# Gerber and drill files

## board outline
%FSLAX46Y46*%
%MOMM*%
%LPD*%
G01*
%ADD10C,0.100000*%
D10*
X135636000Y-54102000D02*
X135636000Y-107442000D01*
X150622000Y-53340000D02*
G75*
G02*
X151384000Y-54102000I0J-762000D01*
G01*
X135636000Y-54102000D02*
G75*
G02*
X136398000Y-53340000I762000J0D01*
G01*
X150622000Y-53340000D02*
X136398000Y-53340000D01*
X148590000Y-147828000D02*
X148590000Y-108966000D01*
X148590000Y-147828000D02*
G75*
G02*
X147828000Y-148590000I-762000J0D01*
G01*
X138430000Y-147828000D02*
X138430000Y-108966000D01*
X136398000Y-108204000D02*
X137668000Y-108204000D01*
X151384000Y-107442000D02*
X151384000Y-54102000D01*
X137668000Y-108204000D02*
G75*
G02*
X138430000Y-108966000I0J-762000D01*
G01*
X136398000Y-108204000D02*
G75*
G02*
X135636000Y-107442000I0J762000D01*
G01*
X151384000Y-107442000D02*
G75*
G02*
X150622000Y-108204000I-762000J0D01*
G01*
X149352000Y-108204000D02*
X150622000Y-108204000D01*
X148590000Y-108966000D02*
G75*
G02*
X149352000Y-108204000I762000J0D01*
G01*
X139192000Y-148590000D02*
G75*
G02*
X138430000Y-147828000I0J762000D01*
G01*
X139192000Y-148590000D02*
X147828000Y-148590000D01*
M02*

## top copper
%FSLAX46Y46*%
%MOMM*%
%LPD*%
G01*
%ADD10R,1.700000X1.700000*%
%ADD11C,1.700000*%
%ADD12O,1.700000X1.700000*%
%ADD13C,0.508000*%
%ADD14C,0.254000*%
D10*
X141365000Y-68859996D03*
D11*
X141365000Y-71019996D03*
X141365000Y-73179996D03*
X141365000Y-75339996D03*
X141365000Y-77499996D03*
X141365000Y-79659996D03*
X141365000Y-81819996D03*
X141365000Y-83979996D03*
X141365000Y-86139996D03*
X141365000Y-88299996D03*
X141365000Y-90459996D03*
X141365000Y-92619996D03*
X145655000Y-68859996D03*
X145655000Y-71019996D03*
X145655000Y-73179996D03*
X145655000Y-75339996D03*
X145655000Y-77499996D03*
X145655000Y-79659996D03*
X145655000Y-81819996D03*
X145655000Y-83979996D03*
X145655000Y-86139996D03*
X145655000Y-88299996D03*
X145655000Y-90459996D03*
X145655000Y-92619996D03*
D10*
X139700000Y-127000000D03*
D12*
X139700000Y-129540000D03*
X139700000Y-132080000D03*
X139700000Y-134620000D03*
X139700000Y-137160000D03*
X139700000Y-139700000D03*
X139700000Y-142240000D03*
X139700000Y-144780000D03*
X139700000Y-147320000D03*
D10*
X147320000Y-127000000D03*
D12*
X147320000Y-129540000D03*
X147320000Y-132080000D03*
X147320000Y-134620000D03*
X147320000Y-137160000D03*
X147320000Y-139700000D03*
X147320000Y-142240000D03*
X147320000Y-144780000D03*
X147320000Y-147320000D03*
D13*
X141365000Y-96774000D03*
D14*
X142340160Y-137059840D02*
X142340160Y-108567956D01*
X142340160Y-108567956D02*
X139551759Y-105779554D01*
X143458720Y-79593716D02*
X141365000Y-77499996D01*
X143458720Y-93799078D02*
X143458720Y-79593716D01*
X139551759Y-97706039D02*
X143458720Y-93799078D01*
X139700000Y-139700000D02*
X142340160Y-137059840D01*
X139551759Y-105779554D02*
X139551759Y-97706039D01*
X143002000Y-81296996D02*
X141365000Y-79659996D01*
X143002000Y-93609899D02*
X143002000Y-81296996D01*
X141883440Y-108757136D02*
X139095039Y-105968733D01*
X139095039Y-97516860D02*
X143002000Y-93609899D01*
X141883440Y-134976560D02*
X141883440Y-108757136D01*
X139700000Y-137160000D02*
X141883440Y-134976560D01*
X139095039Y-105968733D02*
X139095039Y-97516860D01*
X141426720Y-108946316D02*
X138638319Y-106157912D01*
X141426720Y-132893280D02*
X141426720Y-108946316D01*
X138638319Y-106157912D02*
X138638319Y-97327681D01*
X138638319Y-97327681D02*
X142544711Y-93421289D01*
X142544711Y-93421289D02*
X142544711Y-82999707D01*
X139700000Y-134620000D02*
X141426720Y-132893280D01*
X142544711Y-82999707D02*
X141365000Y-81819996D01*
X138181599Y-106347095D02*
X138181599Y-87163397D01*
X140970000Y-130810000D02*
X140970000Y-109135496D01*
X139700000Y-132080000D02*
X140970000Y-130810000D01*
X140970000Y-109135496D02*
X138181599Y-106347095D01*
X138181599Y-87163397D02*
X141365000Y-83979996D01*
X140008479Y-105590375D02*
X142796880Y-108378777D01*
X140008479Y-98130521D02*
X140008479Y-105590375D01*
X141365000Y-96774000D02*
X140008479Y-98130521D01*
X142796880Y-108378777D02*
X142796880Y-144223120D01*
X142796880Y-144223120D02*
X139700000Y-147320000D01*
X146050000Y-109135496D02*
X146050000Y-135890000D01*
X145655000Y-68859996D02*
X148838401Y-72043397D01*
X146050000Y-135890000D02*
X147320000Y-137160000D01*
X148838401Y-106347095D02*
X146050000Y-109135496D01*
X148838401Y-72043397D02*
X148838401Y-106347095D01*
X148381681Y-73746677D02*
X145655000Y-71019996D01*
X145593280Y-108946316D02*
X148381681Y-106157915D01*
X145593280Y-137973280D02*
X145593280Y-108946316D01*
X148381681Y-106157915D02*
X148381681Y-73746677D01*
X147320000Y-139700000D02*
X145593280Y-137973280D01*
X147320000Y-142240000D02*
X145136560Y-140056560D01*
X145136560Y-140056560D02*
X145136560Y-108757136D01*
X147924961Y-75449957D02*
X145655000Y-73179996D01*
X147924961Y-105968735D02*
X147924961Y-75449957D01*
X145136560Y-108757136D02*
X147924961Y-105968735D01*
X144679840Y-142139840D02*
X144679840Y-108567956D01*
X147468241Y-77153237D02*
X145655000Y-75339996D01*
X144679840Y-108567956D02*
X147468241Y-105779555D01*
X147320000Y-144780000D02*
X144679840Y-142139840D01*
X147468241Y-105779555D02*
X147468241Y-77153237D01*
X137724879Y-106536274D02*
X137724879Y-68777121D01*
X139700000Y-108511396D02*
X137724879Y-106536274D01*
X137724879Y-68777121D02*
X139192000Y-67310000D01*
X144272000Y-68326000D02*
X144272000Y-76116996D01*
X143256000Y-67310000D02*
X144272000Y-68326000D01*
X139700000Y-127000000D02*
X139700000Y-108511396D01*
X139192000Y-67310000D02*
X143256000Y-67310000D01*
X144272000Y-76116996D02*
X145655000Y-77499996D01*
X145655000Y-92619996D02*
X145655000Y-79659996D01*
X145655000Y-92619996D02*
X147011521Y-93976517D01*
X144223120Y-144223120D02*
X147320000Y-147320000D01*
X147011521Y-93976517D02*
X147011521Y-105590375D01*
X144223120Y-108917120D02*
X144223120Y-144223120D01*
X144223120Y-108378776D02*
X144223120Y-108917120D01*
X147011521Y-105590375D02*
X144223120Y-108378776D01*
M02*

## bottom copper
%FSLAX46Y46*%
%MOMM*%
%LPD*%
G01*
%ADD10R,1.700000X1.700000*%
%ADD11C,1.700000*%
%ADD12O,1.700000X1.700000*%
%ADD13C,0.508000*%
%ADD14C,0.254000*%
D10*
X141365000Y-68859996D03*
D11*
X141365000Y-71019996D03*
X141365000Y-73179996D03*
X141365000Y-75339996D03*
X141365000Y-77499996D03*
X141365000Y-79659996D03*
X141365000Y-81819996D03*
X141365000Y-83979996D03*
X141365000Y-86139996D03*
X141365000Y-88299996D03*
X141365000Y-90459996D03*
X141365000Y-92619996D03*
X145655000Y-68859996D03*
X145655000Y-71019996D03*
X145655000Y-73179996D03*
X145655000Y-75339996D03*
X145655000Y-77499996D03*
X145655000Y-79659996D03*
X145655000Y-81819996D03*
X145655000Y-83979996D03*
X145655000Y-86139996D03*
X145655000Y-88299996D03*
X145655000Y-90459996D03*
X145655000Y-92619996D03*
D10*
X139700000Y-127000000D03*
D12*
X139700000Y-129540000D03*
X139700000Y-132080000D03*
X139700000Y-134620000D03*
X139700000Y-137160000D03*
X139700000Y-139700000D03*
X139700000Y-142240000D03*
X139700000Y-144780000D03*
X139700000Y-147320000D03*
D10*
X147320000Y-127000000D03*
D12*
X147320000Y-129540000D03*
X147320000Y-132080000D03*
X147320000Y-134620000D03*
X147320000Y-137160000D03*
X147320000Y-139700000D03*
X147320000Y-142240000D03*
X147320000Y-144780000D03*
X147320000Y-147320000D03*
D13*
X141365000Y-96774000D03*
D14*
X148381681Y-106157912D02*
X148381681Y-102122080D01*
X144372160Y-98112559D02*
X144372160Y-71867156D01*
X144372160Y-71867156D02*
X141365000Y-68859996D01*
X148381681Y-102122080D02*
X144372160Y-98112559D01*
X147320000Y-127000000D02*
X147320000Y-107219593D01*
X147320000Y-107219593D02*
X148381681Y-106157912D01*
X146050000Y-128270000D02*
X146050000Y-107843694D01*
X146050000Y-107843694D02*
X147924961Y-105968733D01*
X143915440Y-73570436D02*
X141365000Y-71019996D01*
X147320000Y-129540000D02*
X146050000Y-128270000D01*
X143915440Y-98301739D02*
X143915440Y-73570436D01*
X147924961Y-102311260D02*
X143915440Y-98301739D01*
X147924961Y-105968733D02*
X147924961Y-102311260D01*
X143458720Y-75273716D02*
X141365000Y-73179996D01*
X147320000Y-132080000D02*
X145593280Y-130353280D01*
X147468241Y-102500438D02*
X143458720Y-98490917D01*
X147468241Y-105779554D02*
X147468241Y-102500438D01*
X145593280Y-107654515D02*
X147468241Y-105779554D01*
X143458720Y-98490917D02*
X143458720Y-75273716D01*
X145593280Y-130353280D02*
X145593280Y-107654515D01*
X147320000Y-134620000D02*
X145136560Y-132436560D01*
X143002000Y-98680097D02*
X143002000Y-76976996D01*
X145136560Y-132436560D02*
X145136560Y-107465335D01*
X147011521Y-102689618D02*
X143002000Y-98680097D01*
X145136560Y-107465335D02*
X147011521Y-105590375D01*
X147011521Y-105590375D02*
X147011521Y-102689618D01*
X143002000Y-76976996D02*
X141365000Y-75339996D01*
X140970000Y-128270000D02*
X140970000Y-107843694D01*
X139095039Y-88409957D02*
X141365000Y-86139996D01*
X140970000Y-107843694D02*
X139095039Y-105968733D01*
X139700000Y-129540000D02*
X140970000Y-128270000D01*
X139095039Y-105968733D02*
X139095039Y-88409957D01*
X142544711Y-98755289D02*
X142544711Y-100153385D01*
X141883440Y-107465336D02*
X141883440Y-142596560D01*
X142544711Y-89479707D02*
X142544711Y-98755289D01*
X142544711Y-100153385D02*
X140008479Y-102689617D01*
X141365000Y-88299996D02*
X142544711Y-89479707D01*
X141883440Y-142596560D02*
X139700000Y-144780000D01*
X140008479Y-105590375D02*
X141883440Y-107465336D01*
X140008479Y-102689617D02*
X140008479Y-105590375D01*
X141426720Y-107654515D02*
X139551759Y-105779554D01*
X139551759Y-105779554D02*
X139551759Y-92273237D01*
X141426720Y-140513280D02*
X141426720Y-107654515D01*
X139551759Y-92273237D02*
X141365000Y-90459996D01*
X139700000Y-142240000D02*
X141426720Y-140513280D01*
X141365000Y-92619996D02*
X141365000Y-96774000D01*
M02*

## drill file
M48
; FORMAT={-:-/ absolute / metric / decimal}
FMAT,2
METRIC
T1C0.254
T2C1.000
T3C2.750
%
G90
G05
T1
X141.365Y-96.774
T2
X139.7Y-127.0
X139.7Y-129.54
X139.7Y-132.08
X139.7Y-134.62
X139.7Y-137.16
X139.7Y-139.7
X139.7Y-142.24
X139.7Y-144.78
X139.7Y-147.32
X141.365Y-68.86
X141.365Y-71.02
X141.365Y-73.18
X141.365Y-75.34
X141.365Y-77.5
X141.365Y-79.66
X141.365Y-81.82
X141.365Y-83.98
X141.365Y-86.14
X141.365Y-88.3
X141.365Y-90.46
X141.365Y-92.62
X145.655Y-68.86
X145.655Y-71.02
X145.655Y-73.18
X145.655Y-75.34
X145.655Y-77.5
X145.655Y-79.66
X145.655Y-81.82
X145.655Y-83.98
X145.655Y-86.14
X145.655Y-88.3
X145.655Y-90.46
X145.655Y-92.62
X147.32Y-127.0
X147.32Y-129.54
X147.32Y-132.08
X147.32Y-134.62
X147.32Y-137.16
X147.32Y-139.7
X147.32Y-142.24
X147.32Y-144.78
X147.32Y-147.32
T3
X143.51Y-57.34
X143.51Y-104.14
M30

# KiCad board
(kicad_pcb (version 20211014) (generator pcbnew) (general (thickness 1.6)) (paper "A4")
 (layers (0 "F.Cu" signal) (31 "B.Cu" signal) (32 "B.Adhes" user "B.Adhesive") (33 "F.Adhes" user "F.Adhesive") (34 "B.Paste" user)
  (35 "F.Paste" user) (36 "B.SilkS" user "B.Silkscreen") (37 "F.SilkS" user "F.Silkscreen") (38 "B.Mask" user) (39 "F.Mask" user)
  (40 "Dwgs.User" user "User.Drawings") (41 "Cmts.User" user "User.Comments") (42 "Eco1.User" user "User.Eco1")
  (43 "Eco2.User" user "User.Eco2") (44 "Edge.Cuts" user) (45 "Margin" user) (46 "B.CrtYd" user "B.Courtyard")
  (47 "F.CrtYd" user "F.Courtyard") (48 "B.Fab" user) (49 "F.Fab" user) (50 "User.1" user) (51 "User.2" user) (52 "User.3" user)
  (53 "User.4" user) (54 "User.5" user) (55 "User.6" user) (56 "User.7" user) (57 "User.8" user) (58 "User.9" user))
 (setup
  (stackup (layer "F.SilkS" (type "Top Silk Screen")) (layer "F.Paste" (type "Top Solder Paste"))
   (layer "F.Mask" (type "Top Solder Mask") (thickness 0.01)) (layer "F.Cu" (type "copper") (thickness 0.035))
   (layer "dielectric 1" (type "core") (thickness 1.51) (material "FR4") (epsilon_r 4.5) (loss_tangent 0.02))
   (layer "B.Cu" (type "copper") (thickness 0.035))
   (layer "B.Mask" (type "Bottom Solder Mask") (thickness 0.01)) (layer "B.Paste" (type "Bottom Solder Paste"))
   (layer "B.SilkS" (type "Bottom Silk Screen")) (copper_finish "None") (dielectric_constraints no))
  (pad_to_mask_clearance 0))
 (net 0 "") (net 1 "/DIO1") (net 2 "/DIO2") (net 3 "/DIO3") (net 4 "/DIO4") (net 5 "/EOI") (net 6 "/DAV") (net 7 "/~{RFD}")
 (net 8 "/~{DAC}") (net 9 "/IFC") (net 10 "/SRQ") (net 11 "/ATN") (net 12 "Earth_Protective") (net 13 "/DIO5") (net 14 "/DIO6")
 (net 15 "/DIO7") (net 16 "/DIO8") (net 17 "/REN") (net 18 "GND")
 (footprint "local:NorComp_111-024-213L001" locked (layer "F.Cu") (at 143.51 80.739996 90)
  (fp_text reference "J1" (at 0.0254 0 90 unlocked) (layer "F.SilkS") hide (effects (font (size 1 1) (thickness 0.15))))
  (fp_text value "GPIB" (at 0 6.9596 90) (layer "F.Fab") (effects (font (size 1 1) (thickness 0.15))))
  (pad "" np_thru_hole circle locked (at -23.4 0 90) (size 2.75 2.75) (drill 2.75) (layers *.Cu *.Mask) (solder_mask_margin 1.75)
   (clearance 2))
  (pad "" np_thru_hole circle locked (at 23.4 0 90) (size 2.75 2.75) (drill 2.75) (layers *.Cu *.Mask) (solder_mask_margin 1.75)
   (clearance 2))
  (pad "1" thru_hole rect locked (at 11.88 -2.145 90) (size 1.7 1.7) (drill 1) (layers *.Cu *.Mask) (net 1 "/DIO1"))
  (pad "2" thru_hole circle locked (at 9.72 -2.145 90) (size 1.7 1.7) (drill 1) (layers *.Cu *.Mask) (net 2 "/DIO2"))
  (pad "3" thru_hole circle locked (at 7.56 -2.145 90) (size 1.7 1.7) (drill 1) (layers *.Cu *.Mask) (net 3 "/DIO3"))
  (pad "4" thru_hole circle locked (at 5.4 -2.145 90) (size 1.7 1.7) (drill 1) (layers *.Cu *.Mask) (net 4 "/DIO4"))
  (pad "5" thru_hole circle locked (at 3.24 -2.145 90) (size 1.7 1.7) (drill 1) (layers *.Cu *.Mask) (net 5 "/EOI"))
  (pad "6" thru_hole circle locked (at 1.08 -2.145 90) (size 1.7 1.7) (drill 1) (layers *.Cu *.Mask) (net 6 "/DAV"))
  (pad "7" thru_hole circle locked (at -1.08 -2.145 90) (size 1.7 1.7) (drill 1) (layers *.Cu *.Mask) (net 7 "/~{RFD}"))
  (pad "8" thru_hole circle locked (at -3.24 -2.145 90) (size 1.7 1.7) (drill 1) (layers *.Cu *.Mask) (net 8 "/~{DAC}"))
  (pad "9" thru_hole circle locked (at -5.4 -2.145 90) (size 1.7 1.7) (drill 1) (layers *.Cu *.Mask) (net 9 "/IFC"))
  (pad "10" thru_hole circle locked (at -7.56 -2.145 90) (size 1.7 1.7) (drill 1) (layers *.Cu *.Mask) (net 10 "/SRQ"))
  (pad "11" thru_hole circle locked (at -9.72 -2.145 90) (size 1.7 1.7) (drill 1) (layers *.Cu *.Mask) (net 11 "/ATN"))
  (pad "12" thru_hole circle locked (at -11.88 -2.145 90) (size 1.7 1.7) (drill 1) (layers *.Cu *.Mask) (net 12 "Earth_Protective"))
  (pad "13" thru_hole circle locked (at 11.88 2.145 90) (size 1.7 1.7) (drill 1) (layers *.Cu *.Mask) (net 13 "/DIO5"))
  (pad "14" thru_hole circle locked (at 9.72 2.145 90) (size 1.7 1.7) (drill 1) (layers *.Cu *.Mask) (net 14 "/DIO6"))
  (pad "15" thru_hole circle locked (at 7.56 2.145 90) (size 1.7 1.7) (drill 1) (layers *.Cu *.Mask) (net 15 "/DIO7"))
  (pad "16" thru_hole circle locked (at 5.4 2.145 90) (size 1.7 1.7) (drill 1) (layers *.Cu *.Mask) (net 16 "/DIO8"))
  (pad "17" thru_hole circle locked (at 3.24 2.145 90) (size 1.7 1.7) (drill 1) (layers *.Cu *.Mask) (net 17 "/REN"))
  (pad "18" thru_hole circle locked (at 1.08 2.145 90) (size 1.7 1.7) (drill 1) (layers *.Cu *.Mask) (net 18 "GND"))
  (pad "19" thru_hole circle locked (at -1.08 2.145 90) (size 1.7 1.7) (drill 1) (layers *.Cu *.Mask) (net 18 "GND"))
  (pad "20" thru_hole circle locked (at -3.24 2.145 90) (size 1.7 1.7) (drill 1) (layers *.Cu *.Mask) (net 18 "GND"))
  (pad "21" thru_hole circle locked (at -5.4 2.145 90) (size 1.7 1.7) (drill 1) (layers *.Cu *.Mask) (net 18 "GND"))
  (pad "22" thru_hole circle locked (at -7.56 2.145 90) (size 1.7 1.7) (drill 1) (layers *.Cu *.Mask) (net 18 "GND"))
  (pad "23" thru_hole circle locked (at -9.72 2.145 90) (size 1.7 1.7) (drill 1) (layers *.Cu *.Mask) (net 18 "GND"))
  (pad "24" thru_hole circle locked (at -11.88 2.145 90) (size 1.7 1.7) (drill 1) (layers *.Cu *.Mask) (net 18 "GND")))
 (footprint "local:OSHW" (layer "F.Cu") (at 142.24 122.936 90)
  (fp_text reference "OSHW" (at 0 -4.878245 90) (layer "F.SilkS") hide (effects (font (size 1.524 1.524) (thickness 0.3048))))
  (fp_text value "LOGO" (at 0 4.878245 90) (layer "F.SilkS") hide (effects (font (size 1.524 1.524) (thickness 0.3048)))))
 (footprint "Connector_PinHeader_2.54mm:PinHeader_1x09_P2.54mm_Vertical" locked (layer "B.Cu") (at 139.7 127 180)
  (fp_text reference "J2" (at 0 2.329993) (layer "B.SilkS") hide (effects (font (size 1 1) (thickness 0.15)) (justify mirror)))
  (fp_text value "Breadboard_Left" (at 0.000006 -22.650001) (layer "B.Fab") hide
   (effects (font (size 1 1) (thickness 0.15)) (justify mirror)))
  (pad "1" thru_hole rect locked (at 0 0 180) (size 1.7 1.7) (drill 1) (layers *.Cu *.Mask) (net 17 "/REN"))
  (pad "2" thru_hole oval locked (at 0 -2.54 180) (size 1.7 1.7) (drill 1) (layers *.Cu *.Mask) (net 9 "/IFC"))
  (pad "3" thru_hole oval locked (at 0 -5.08 180) (size 1.7 1.7) (drill 1) (layers *.Cu *.Mask) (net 8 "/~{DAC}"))
  (pad "4" thru_hole oval locked (at 0 -7.62 180) (size 1.7 1.7) (drill 1) (layers *.Cu *.Mask) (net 7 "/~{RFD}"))
  (pad "5" thru_hole oval locked (at 0 -10.16 180) (size 1.7 1.7) (drill 1) (layers *.Cu *.Mask) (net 6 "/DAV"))
  (pad "6" thru_hole oval locked (at 0 -12.7 180) (size 1.7 1.7) (drill 1) (layers *.Cu *.Mask) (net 5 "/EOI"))
  (pad "7" thru_hole oval locked (at 0 -15.24 180) (size 1.7 1.7) (drill 1) (layers *.Cu *.Mask) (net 11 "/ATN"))
  (pad "8" thru_hole oval locked (at 0 -17.78 180) (size 1.7 1.7) (drill 1) (layers *.Cu *.Mask) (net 10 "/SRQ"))
  (pad "9" thru_hole oval locked (at 0 -20.32 180) (size 1.7 1.7) (drill 1) (layers *.Cu *.Mask) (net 12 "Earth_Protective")))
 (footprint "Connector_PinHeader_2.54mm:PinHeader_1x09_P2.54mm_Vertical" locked (layer "B.Cu") (at 147.32 127 180)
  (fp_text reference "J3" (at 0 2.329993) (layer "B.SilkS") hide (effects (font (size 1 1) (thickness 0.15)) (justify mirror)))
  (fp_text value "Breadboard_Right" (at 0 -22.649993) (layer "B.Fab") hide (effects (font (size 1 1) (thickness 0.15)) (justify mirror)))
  (pad "1" thru_hole rect locked (at 0 0 180) (size 1.7 1.7) (drill 1) (layers *.Cu *.Mask) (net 1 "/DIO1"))
  (pad "2" thru_hole oval locked (at 0 -2.54 180) (size 1.7 1.7) (drill 1) (layers *.Cu *.Mask) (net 2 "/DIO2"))
  (pad "3" thru_hole oval locked (at 0 -5.08 180) (size 1.7 1.7) (drill 1) (layers *.Cu *.Mask) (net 3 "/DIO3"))
  (pad "4" thru_hole oval locked (at 0 -7.62 180) (size 1.7 1.7) (drill 1) (layers *.Cu *.Mask) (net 4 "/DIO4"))
  (pad "5" thru_hole oval locked (at 0 -10.16 180) (size 1.7 1.7) (drill 1) (layers *.Cu *.Mask) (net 13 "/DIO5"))
  (pad "6" thru_hole oval locked (at 0 -12.7 180) (size 1.7 1.7) (drill 1) (layers *.Cu *.Mask) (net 14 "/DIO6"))
  (pad "7" thru_hole oval locked (at 0 -15.24 180) (size 1.7 1.7) (drill 1) (layers *.Cu *.Mask) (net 15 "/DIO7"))
  (pad "8" thru_hole oval locked (at 0 -17.78 180) (size 1.7 1.7) (drill 1) (layers *.Cu *.Mask) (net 16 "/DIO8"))
  (pad "9" thru_hole oval locked (at 0 -20.32 180) (size 1.7 1.7) (drill 1) (layers *.Cu *.Mask) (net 18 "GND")))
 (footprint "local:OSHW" (layer "B.Cu") (at 144.78 122.936 90)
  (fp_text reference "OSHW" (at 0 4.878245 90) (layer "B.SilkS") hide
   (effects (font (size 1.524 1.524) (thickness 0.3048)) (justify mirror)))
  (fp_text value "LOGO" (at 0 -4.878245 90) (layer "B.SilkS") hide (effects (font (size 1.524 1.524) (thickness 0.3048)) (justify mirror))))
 (gr_line (start 135.636 54.102) (end 135.636 107.442) (layer "Edge.Cuts") (width 0.1))
 (gr_arc (start 150.622 53.34) (mid 151.160815 53.563185) (end 151.384 54.102) (layer "Edge.Cuts") (width 0.1))
 (gr_arc (start 135.636 54.102) (mid 135.859185 53.563185) (end 136.398 53.34) (layer "Edge.Cuts") (width 0.1))
 (gr_line (start 150.622 53.34) (end 136.398 53.34) (layer "Edge.Cuts") (width 0.1))
 (gr_line (start 148.59 147.828) (end 148.59 108.966) (layer "Edge.Cuts") (width 0.1))
 (gr_arc (start 148.59 147.828) (mid 148.366815 148.366815) (end 147.828 148.59) (layer "Edge.Cuts") (width 0.1))
 (gr_line (start 138.43 147.828) (end 138.43 108.966) (layer "Edge.Cuts") (width 0.1))
 (gr_line (start 136.398 108.204) (end 137.668 108.204) (layer "Edge.Cuts") (width 0.1))
 (gr_line (start 151.384 107.442) (end 151.384 54.102) (layer "Edge.Cuts") (width 0.1))
 (gr_arc (start 137.668 108.204) (mid 138.206815 108.427185) (end 138.43 108.966) (layer "Edge.Cuts") (width 0.1))
 (gr_arc (start 136.398 108.204) (mid 135.859185 107.980815) (end 135.636 107.442) (layer "Edge.Cuts") (width 0.1))
 (gr_arc (start 151.384 107.442) (mid 151.160815 107.980815) (end 150.622 108.204) (layer "Edge.Cuts") (width 0.1))
 (gr_line (start 149.352 108.204) (end 150.622 108.204) (layer "Edge.Cuts") (width 0.1))
 (gr_arc (start 148.59 108.966) (mid 148.813185 108.427185) (end 149.352 108.204) (layer "Edge.Cuts") (width 0.1))
 (gr_arc (start 139.192 148.59) (mid 138.653185 148.366815) (end 138.43 147.828) (layer "Edge.Cuts") (width 0.1))
 (gr_line (start 139.192 148.59) (end 147.828 148.59) (layer "Edge.Cuts") (width 0.1))
 (segment (start 148.381681 106.157912) (end 148.381681 102.12208) (width 0.254) (layer "B.Cu") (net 1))
 (segment (start 144.37216 98.112559) (end 144.37216 71.867156) (width 0.254) (layer "B.Cu") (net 1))
 (segment (start 144.37216 71.867156) (end 141.365 68.859996) (width 0.254) (layer "B.Cu") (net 1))
 (segment (start 148.381681 102.12208) (end 144.37216 98.112559) (width 0.254) (layer "B.Cu") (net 1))
 (segment (start 147.32 127) (end 147.32 107.219593) (width 0.254) (layer "B.Cu") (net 1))
 (segment (start 147.32 107.219593) (end 148.381681 106.157912) (width 0.254) (layer "B.Cu") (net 1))
 (segment (start 146.05 128.27) (end 146.05 107.843694) (width 0.254) (layer "B.Cu") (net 2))
 (segment (start 146.05 107.843694) (end 147.924961 105.968733) (width 0.254) (layer "B.Cu") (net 2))
 (segment (start 143.91544 73.570436) (end 141.365 71.019996) (width 0.254) (layer "B.Cu") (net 2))
 (segment (start 147.32 129.54) (end 146.05 128.27) (width 0.254) (layer "B.Cu") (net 2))
 (segment (start 143.91544 98.301739) (end 143.91544 73.570436) (width 0.254) (layer "B.Cu") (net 2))
 (segment (start 147.924961 102.31126) (end 143.91544 98.301739) (width 0.254) (layer "B.Cu") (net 2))
 (segment (start 147.924961 105.968733) (end 147.924961 102.31126) (width 0.254) (layer "B.Cu") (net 2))
 (segment (start 143.45872 75.273716) (end 141.365 73.179996) (width 0.254) (layer "B.Cu") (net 3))
 (segment (start 147.32 132.08) (end 145.59328 130.35328) (width 0.254) (layer "B.Cu") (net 3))
 (segment (start 147.468241 102.500438) (end 143.45872 98.490917) (width 0.254) (layer "B.Cu") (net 3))
 (segment (start 147.468241 105.779554) (end 147.468241 102.500438) (width 0.254) (layer "B.Cu") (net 3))
 (segment (start 145.59328 107.654515) (end 147.468241 105.779554) (width 0.254) (layer "B.Cu") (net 3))
 (segment (start 143.45872 98.490917) (end 143.45872 75.273716) (width 0.254) (layer "B.Cu") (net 3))
 (segment (start 145.59328 130.35328) (end 145.59328 107.654515) (width 0.254) (layer "B.Cu") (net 3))
 (segment (start 147.32 134.62) (end 145.13656 132.43656) (width 0.254) (layer "B.Cu") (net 4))
 (segment (start 143.002 98.680097) (end 143.002 76.976996) (width 0.254) (layer "B.Cu") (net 4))
 (segment (start 145.13656 132.43656) (end 145.13656 107.465335) (width 0.254) (layer "B.Cu") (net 4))
 (segment (start 147.011521 102.689618) (end 143.002 98.680097) (width 0.254) (layer "B.Cu") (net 4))
 (segment (start 145.13656 107.465335) (end 147.011521 105.590375) (width 0.254) (layer "B.Cu") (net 4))
 (segment (start 147.011521 105.590375) (end 147.011521 102.689618) (width 0.254) (layer "B.Cu") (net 4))
 (segment (start 143.002 76.976996) (end 141.365 75.339996) (width 0.254) (layer "B.Cu") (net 4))
 (segment (start 142.34016 137.05984) (end 142.34016 108.567956) (width 0.254) (layer "F.Cu") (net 5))
 (segment (start 142.34016 108.567956) (end 139.551759 105.779554) (width 0.254) (layer "F.Cu") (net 5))
 (segment (start 143.45872 79.593716) (end 141.365 77.499996) (width 0.254) (layer "F.Cu") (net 5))
 (segment (start 143.45872 93.799078) (end 143.45872 79.593716) (width 0.254) (layer "F.Cu") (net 5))
 (segment (start 139.551759 97.706039) (end 143.45872 93.799078) (width 0.254) (layer "F.Cu") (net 5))
 (segment (start 139.7 139.7) (end 142.34016 137.05984) (width 0.254) (layer "F.Cu") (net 5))
 (segment (start 139.551759 105.779554) (end 139.551759 97.706039) (width 0.254) (layer "F.Cu") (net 5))
 (segment (start 143.002 81.296996) (end 141.365 79.659996) (width 0.254) (layer "F.Cu") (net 6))
 (segment (start 143.002 93.609899) (end 143.002 81.296996) (width 0.254) (layer "F.Cu") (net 6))
 (segment (start 141.88344 108.757136) (end 139.095039 105.968733) (width 0.254) (layer "F.Cu") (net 6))
 (segment (start 139.095039 97.51686) (end 143.002 93.609899) (width 0.254) (layer "F.Cu") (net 6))
 (segment (start 141.88344 134.97656) (end 141.88344 108.757136) (width 0.254) (layer "F.Cu") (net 6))
 (segment (start 139.7 137.16) (end 141.88344 134.97656) (width 0.254) (layer "F.Cu") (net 6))
 (segment (start 139.095039 105.968733) (end 139.095039 97.51686) (width 0.254) (layer "F.Cu") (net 6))
 (segment (start 141.42672 108.946316) (end 138.638319 106.157912) (width 0.254) (layer "F.Cu") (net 7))
 (segment (start 141.42672 132.89328) (end 141.42672 108.946316) (width 0.254) (layer "F.Cu") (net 7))
 (segment (start 138.638319 106.157912) (end 138.638319 97.327681) (width 0.254) (layer "F.Cu") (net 7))
 (segment (start 138.638319 97.327681) (end 142.544711 93.421289) (width 0.254) (layer "F.Cu") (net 7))
 (segment (start 142.544711 93.421289) (end 142.544711 82.999707) (width 0.254) (layer "F.Cu") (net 7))
 (segment (start 139.7 134.62) (end 141.42672 132.89328) (width 0.254) (layer "F.Cu") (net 7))
 (segment (start 142.544711 82.999707) (end 141.365 81.819996) (width 0.254) (layer "F.Cu") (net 7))
 (segment (start 138.181599 106.347095) (end 138.181599 87.163397) (width 0.254) (layer "F.Cu") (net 8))
 (segment (start 140.97 130.81) (end 140.97 109.135496) (width 0.254) (layer "F.Cu") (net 8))
 (segment (start 139.7 132.08) (end 140.97 130.81) (width 0.254) (layer "F.Cu") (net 8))
 (segment (start 140.97 109.135496) (end 138.181599 106.347095) (width 0.254) (layer "F.Cu") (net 8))
 (segment (start 138.181599 87.163397) (end 141.365 83.979996) (width 0.254) (layer "F.Cu") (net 8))
 (segment (start 140.97 128.27) (end 140.97 107.843694) (width 0.254) (layer "B.Cu") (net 9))
 (segment (start 139.095039 88.409957) (end 141.365 86.139996) (width 0.254) (layer "B.Cu") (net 9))
 (segment (start 140.97 107.843694) (end 139.095039 105.968733) (width 0.254) (layer "B.Cu") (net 9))
 (segment (start 139.7 129.54) (end 140.97 128.27) (width 0.254) (layer "B.Cu") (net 9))
 (segment (start 139.095039 105.968733) (end 139.095039 88.409957) (width 0.254) (layer "B.Cu") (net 9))
 (segment (start 142.544711 98.755289) (end 142.544711 100.153385) (width 0.254) (layer "B.Cu") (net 10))
 (segment (start 141.88344 107.465336) (end 141.88344 142.59656) (width 0.254) (layer "B.Cu") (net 10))
 (segment (start 142.544711 89.479707) (end 142.544711 98.755289) (width 0.254) (layer "B.Cu") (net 10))
 (segment (start 142.544711 100.153385) (end 140.008479 102.689617) (width 0.254) (layer "B.Cu") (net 10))
 (segment (start 141.365 88.299996) (end 142.544711 89.479707) (width 0.254) (layer "B.Cu") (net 10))
 (segment (start 141.88344 142.59656) (end 139.7 144.78) (width 0.254) (layer "B.Cu") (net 10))
 (segment (start 140.008479 105.590375) (end 141.88344 107.465336) (width 0.254) (layer "B.Cu") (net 10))
 (segment (start 140.008479 102.689617) (end 140.008479 105.590375) (width 0.254) (layer "B.Cu") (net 10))
 (segment (start 141.42672 107.654515) (end 139.551759 105.779554) (width 0.254) (layer "B.Cu") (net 11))
 (segment (start 139.551759 105.779554) (end 139.551759 92.273237) (width 0.254) (layer "B.Cu") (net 11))
 (segment (start 141.42672 140.51328) (end 141.42672 107.654515) (width 0.254) (layer "B.Cu") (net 11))
 (segment (start 139.551759 92.273237) (end 141.365 90.459996) (width 0.254) (layer "B.Cu") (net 11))
 (segment (start 139.7 142.24) (end 141.42672 140.51328) (width 0.254) (layer "B.Cu") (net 11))
 (segment (start 140.008479 105.590375) (end 142.79688 108.378777) (width 0.254) (layer "F.Cu") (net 12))
 (segment (start 140.008479 98.130521) (end 140.008479 105.590375) (width 0.254) (layer "F.Cu") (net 12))
 (segment (start 141.365 96.774) (end 140.008479 98.130521) (width 0.254) (layer "F.Cu") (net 12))
 (segment (start 142.79688 108.378777) (end 142.79688 144.22312) (width 0.254) (layer "F.Cu") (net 12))
 (segment (start 142.79688 144.22312) (end 139.7 147.32) (width 0.254) (layer "F.Cu") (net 12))
 (via (at 141.365 96.774) (size 0.508) (drill 0.254) (layers "F.Cu" "B.Cu") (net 12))
 (segment (start 141.365 92.619996) (end 141.365 96.774) (width 0.254) (layer "B.Cu") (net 12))
 (segment (start 146.05 109.135496) (end 146.05 135.89) (width 0.254) (layer "F.Cu") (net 13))
 (segment (start 145.655 68.859996) (end 148.838401 72.043397) (width 0.254) (layer "F.Cu") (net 13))
 (segment (start 146.05 135.89) (end 147.32 137.16) (width 0.254) (layer "F.Cu") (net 13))
 (segment (start 148.838401 106.347095) (end 146.05 109.135496) (width 0.254) (layer "F.Cu") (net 13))
 (segment (start 148.838401 72.043397) (end 148.838401 106.347095) (width 0.254) (layer "F.Cu") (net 13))
 (segment (start 148.381681 73.746677) (end 145.655 71.019996) (width 0.254) (layer "F.Cu") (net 14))
 (segment (start 145.59328 108.946316) (end 148.381681 106.157915) (width 0.254) (layer "F.Cu") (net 14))
 (segment (start 145.59328 137.97328) (end 145.59328 108.946316) (width 0.254) (layer "F.Cu") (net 14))
 (segment (start 148.381681 106.157915) (end 148.381681 73.746677) (width 0.254) (layer "F.Cu") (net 14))
 (segment (start 147.32 139.7) (end 145.59328 137.97328) (width 0.254) (layer "F.Cu") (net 14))
 (segment (start 147.32 142.24) (end 145.13656 140.05656) (width 0.254) (layer "F.Cu") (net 15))
 (segment (start 145.13656 140.05656) (end 145.13656 108.757136) (width 0.254) (layer "F.Cu") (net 15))
 (segment (start 147.924961 75.449957) (end 145.655 73.179996) (width 0.254) (layer "F.Cu") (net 15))
 (segment (start 147.924961 105.968735) (end 147.924961 75.449957) (width 0.254) (layer "F.Cu") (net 15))
 (segment (start 145.13656 108.757136) (end 147.924961 105.968735) (width 0.254) (layer "F.Cu") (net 15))
 (segment (start 144.67984 142.13984) (end 144.67984 108.567956) (width 0.254) (layer "F.Cu") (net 16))
 (segment (start 147.468241 77.153237) (end 145.655 75.339996) (width 0.254) (layer "F.Cu") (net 16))
 (segment (start 144.67984 108.567956) (end 147.468241 105.779555) (width 0.254) (layer "F.Cu") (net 16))
 (segment (start 147.32 144.78) (end 144.67984 142.13984) (width 0.254) (layer "F.Cu") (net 16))
 (segment (start 147.468241 105.779555) (end 147.468241 77.153237) (width 0.254) (layer "F.Cu") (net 16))
 (segment (start 137.724879 106.536274) (end 137.724879 68.777121) (width 0.254) (layer "F.Cu") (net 17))
 (segment (start 139.7 108.511396) (end 137.724879 106.536274) (width 0.254) (layer "F.Cu") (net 17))
 (segment (start 137.724879 68.777121) (end 139.192 67.31) (width 0.254) (layer "F.Cu") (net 17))
 (segment (start 144.272 68.326) (end 144.272 76.116996) (width 0.254) (layer "F.Cu") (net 17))
 (segment (start 143.256 67.31) (end 144.272 68.326) (width 0.254) (layer "F.Cu") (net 17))
 (segment (start 139.7 127) (end 139.7 108.511396) (width 0.254) (layer "F.Cu") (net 17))
 (segment (start 139.192 67.31) (end 143.256 67.31) (width 0.254) (layer "F.Cu") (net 17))
 (segment (start 144.272 76.116996) (end 145.655 77.499996) (width 0.254) (layer "F.Cu") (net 17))
 (segment (start 145.655 92.619996) (end 145.655 79.659996) (width 0.254) (layer "F.Cu") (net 18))
 (segment (start 145.655 92.619996) (end 147.011521 93.976517) (width 0.254) (layer "F.Cu") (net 18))
 (segment (start 144.22312 144.22312) (end 147.32 147.32) (width 0.254) (layer "F.Cu") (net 18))
 (segment (start 147.011521 93.976517) (end 147.011521 105.590375) (width 0.254) (layer "F.Cu") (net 18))
 (segment (start 144.22312 108.91712) (end 144.22312 144.22312) (width 0.254) (layer "F.Cu") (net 18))
 (segment (start 144.22312 108.378776) (end 144.22312 108.91712) (width 0.254) (layer "F.Cu") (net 18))
 (segment (start 147.011521 105.590375) (end 144.22312 108.378776) (width 0.254) (layer "F.Cu") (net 18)))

